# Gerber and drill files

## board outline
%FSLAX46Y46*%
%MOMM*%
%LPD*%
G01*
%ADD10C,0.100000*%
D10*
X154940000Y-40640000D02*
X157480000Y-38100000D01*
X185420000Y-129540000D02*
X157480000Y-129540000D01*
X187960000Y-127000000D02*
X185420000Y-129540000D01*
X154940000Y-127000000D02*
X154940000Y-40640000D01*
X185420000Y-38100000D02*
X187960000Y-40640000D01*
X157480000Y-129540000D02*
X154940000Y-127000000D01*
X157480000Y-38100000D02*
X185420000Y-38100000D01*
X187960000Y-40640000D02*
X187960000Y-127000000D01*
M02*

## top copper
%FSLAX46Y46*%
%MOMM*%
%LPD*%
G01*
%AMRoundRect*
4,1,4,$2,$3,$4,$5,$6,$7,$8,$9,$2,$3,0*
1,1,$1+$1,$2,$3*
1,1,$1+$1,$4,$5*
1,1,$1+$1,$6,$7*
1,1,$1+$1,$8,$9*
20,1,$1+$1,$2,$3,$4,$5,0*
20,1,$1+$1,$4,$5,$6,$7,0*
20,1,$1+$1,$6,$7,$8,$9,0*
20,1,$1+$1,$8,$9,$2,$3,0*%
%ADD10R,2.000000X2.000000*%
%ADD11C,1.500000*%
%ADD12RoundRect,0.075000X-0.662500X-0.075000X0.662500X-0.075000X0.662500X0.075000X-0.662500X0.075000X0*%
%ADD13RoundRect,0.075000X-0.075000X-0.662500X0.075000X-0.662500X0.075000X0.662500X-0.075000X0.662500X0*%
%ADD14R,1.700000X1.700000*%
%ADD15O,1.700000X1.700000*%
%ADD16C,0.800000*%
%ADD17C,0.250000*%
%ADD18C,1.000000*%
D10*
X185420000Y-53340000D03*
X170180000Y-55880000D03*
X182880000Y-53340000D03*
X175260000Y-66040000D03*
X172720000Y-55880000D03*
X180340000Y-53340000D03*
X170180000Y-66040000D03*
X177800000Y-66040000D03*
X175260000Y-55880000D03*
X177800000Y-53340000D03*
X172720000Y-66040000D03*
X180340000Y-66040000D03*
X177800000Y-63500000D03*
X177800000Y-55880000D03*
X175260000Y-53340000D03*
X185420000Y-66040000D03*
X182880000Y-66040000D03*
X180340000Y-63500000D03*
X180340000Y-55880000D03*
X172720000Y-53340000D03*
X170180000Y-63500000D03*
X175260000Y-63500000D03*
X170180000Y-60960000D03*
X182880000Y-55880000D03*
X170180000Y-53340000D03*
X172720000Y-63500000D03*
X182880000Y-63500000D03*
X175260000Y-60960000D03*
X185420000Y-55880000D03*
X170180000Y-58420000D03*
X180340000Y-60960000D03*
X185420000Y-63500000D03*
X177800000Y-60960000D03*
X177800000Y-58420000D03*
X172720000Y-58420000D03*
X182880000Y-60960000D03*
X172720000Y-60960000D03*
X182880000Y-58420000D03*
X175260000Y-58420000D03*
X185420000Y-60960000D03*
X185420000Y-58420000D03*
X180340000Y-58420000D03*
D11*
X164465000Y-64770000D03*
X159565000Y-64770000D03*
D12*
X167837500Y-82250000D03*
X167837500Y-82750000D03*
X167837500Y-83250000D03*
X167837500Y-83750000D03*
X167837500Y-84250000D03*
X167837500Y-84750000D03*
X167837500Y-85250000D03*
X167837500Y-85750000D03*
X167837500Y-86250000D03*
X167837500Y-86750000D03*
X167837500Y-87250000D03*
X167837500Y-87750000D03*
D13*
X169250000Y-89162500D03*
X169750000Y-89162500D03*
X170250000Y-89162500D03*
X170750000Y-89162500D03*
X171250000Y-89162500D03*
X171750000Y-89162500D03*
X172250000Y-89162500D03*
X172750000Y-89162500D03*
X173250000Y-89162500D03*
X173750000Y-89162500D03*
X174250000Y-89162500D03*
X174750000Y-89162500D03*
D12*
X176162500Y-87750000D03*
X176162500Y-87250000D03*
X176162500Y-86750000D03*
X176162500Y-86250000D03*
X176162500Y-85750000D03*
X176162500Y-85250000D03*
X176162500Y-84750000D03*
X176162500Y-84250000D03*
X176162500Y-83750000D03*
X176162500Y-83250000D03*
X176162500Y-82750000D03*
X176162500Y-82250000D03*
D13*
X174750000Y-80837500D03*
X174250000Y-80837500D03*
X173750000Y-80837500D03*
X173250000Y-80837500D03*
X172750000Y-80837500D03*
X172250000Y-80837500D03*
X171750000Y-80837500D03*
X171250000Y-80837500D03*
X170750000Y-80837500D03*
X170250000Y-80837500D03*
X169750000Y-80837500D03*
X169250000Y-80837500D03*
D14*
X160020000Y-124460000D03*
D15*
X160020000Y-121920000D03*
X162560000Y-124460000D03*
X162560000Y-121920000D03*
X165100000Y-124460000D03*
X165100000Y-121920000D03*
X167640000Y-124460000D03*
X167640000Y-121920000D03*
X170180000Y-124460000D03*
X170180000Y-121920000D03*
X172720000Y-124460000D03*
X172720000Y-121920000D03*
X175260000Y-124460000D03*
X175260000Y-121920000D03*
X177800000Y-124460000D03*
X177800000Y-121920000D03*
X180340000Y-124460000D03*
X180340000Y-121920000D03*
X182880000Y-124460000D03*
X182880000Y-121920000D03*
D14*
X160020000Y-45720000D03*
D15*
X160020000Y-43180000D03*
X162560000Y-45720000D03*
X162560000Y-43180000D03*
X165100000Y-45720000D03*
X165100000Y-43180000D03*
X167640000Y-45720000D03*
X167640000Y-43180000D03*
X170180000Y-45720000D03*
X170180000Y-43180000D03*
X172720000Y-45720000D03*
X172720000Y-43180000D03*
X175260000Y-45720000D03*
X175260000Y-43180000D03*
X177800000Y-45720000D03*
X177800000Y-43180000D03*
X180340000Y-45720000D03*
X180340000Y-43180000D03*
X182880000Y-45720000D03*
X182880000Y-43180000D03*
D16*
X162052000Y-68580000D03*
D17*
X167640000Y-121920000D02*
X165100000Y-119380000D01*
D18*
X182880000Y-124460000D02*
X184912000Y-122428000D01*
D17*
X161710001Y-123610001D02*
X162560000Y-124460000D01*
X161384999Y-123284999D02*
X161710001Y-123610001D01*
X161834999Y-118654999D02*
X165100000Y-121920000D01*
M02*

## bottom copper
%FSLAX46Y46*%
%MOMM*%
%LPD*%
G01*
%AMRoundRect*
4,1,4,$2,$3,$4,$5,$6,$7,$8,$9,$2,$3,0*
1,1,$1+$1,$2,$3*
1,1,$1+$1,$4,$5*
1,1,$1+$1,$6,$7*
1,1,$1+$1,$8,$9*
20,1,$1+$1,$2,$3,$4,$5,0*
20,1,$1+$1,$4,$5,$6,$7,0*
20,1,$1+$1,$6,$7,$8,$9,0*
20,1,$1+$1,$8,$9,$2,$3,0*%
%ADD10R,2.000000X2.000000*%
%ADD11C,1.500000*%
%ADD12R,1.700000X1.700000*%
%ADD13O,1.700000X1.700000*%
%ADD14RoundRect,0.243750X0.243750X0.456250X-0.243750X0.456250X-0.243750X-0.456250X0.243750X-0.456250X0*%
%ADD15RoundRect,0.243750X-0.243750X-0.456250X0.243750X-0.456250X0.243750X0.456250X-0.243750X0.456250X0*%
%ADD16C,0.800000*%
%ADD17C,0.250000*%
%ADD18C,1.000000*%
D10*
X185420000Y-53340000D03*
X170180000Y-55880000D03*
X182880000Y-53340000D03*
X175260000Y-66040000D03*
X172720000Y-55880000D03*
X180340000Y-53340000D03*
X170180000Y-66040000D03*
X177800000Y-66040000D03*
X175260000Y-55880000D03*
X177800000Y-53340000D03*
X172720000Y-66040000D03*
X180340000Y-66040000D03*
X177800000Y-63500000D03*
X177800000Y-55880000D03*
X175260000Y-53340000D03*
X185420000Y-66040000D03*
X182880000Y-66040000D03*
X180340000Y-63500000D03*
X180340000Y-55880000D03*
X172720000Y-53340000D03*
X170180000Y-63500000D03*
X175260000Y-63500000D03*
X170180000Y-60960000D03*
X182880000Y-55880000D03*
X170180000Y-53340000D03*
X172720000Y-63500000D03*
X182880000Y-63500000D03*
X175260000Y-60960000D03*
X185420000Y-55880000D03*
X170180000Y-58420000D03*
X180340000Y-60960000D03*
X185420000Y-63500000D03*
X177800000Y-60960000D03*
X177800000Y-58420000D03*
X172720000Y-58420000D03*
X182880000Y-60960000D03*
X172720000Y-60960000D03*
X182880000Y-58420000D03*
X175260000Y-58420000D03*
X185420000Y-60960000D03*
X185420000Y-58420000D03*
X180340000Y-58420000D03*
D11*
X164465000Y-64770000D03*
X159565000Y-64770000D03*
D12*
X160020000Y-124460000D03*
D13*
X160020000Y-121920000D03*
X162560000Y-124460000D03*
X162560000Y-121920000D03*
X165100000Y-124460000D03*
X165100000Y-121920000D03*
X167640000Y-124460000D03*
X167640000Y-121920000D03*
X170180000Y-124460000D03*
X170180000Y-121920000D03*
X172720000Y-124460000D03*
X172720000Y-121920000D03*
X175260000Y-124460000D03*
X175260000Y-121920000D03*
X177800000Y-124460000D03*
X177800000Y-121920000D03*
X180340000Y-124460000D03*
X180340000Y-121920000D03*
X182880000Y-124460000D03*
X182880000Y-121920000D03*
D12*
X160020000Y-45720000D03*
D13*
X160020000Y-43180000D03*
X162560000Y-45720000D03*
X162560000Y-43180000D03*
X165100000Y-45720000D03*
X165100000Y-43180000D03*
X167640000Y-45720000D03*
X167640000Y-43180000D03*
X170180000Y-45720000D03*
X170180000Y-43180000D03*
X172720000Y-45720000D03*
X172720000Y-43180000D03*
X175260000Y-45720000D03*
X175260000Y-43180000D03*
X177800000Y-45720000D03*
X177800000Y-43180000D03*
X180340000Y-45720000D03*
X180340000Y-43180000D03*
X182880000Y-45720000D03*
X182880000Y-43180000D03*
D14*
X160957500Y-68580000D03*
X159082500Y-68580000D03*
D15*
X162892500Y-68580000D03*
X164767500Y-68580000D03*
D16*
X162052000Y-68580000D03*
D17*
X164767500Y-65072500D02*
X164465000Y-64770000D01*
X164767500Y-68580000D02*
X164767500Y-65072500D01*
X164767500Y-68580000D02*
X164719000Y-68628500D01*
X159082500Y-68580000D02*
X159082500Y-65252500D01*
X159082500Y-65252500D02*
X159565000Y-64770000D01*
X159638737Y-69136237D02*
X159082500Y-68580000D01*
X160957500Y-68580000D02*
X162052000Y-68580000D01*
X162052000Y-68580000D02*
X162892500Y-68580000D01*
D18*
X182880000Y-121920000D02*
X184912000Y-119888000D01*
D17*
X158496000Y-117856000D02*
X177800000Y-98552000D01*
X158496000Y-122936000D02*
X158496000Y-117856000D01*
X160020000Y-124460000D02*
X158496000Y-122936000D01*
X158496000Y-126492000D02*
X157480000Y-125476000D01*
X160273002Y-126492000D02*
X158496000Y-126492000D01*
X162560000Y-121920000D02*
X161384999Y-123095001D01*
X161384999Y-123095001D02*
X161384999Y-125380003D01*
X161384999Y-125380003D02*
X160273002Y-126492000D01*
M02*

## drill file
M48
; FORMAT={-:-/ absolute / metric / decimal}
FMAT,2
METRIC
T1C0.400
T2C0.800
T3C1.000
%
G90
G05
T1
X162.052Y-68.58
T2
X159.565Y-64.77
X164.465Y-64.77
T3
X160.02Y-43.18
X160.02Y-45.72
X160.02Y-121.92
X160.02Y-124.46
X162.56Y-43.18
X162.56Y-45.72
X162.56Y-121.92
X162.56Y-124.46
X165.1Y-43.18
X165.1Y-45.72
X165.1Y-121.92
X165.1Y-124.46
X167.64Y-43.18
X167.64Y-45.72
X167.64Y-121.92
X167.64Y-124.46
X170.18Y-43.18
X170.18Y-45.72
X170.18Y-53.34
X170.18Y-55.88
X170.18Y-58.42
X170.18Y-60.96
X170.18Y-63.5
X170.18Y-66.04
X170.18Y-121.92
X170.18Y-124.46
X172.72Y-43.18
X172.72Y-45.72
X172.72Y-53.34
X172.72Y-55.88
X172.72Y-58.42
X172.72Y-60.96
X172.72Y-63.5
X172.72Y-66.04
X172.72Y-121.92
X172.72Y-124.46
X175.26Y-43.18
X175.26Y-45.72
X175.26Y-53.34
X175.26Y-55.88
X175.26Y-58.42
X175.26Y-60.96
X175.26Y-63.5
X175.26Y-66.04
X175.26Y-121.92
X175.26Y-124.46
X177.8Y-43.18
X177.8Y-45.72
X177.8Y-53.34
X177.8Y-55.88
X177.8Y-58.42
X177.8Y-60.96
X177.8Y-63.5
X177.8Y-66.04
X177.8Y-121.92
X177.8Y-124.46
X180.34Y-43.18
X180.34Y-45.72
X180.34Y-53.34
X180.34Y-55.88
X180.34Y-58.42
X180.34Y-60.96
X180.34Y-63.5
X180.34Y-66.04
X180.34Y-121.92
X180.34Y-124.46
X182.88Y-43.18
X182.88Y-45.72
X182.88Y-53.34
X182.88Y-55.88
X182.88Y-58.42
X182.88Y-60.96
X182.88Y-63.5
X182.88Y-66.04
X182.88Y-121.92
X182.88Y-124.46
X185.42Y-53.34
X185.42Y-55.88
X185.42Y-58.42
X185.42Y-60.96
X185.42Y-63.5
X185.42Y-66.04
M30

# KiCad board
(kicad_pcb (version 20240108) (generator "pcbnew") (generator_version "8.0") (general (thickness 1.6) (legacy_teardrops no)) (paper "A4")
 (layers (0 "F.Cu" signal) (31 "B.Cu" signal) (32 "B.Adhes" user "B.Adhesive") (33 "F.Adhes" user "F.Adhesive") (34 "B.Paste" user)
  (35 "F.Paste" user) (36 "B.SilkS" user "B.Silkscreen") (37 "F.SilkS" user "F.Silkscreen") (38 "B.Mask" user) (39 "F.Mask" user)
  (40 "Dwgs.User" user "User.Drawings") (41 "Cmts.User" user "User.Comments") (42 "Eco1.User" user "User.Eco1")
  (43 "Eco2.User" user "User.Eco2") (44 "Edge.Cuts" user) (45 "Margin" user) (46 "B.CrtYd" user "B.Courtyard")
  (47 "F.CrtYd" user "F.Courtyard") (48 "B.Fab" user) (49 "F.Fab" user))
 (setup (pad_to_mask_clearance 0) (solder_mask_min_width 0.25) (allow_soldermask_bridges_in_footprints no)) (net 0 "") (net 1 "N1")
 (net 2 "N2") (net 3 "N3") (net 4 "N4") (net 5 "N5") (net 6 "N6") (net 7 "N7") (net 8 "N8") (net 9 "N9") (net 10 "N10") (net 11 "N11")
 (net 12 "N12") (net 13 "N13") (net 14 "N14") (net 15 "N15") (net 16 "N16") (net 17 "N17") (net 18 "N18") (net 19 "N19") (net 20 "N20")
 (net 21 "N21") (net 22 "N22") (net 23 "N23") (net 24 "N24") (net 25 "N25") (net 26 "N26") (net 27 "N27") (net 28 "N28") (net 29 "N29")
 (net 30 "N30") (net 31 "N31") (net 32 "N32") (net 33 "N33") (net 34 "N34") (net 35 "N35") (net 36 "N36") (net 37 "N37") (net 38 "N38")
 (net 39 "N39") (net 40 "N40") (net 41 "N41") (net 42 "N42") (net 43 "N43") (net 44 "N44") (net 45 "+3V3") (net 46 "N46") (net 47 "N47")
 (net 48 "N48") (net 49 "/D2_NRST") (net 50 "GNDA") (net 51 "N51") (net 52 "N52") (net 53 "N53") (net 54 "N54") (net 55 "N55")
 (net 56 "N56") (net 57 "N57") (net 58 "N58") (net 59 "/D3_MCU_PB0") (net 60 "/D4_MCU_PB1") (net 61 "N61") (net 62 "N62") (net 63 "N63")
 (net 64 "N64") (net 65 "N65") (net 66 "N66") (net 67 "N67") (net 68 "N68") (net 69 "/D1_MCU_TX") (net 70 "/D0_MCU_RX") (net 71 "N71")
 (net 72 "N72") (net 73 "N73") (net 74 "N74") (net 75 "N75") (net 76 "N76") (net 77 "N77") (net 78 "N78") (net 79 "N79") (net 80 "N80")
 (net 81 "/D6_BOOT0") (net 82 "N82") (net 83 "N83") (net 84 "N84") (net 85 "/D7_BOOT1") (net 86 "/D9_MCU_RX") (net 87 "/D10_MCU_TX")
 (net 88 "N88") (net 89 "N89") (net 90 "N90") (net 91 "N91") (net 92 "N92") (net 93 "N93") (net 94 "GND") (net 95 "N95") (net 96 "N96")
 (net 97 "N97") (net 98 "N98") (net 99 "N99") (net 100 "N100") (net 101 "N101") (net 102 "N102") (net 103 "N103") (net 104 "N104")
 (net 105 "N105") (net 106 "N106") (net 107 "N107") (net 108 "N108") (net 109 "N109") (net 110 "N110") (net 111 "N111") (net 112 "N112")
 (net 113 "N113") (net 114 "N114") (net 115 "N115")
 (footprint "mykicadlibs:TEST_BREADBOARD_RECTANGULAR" (layer "F.Cu") (at 185.42 53.34)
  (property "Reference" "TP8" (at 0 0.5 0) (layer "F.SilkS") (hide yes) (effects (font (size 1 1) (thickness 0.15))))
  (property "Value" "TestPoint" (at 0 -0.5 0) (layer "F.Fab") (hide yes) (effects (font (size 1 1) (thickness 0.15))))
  (pad "1" thru_hole rect (at 0 0) (size 2 2) (drill 1) (layers "*.Cu" "*.Mask") (remove_unused_layers no) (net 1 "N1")))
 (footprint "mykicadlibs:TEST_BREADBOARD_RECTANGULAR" (layer "F.Cu") (at 170.18 55.88)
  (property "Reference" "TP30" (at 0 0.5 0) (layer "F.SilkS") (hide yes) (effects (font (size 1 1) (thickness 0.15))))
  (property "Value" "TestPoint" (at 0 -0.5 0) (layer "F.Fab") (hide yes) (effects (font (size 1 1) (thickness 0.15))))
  (pad "1" thru_hole rect (at 0 0) (size 2 2) (drill 1) (layers "*.Cu" "*.Mask") (remove_unused_layers no) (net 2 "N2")))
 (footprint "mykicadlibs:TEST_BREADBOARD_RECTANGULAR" (layer "F.Cu") (at 182.88 53.34)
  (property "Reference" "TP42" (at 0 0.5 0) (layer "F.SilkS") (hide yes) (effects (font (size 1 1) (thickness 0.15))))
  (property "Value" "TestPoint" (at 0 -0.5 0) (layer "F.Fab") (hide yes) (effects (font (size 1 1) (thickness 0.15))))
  (pad "1" thru_hole rect (at 0 0) (size 2 2) (drill 1) (layers "*.Cu" "*.Mask") (remove_unused_layers no) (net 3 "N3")))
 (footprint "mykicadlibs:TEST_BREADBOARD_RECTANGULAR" (layer "F.Cu") (at 175.26 66.04)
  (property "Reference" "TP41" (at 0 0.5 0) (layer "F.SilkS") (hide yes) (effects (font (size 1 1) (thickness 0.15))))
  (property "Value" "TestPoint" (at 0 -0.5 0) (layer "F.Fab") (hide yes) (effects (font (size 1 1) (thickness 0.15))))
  (pad "1" thru_hole rect (at 0 0) (size 2 2) (drill 1) (layers "*.Cu" "*.Mask") (remove_unused_layers no) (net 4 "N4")))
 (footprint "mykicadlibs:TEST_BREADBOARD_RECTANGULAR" (layer "F.Cu") (at 172.72 55.88)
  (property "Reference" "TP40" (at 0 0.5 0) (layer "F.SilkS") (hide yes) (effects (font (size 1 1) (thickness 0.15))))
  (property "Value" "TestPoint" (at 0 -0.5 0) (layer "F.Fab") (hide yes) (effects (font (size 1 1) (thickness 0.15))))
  (pad "1" thru_hole rect (at 0 0) (size 2 2) (drill 1) (layers "*.Cu" "*.Mask") (remove_unused_layers no) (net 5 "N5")))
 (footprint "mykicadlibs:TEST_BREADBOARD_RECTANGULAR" (layer "F.Cu") (at 180.34 53.34)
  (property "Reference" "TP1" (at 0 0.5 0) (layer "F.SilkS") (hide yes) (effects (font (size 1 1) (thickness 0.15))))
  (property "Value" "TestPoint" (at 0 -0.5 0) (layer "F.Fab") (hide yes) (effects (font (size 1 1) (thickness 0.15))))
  (pad "1" thru_hole rect (at 0 0) (size 2 2) (drill 1) (layers "*.Cu" "*.Mask") (remove_unused_layers no) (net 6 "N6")))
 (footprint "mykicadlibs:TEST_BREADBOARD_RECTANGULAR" (layer "F.Cu") (at 170.18 66.04)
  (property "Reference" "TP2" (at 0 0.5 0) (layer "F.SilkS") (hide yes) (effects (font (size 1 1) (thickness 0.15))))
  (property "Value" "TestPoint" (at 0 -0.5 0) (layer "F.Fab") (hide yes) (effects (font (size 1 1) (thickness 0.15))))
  (pad "1" thru_hole rect (at 0 0) (size 2 2) (drill 1) (layers "*.Cu" "*.Mask") (remove_unused_layers no) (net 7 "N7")))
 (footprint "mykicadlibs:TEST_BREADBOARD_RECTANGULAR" (layer "F.Cu") (at 177.8 66.04)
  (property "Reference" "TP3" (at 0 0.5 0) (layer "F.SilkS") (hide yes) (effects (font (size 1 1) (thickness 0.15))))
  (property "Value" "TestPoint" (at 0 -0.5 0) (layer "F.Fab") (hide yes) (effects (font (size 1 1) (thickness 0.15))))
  (pad "1" thru_hole rect (at 0 0) (size 2 2) (drill 1) (layers "*.Cu" "*.Mask") (remove_unused_layers no) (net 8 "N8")))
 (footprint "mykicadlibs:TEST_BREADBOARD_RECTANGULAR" (layer "F.Cu") (at 175.26 55.88)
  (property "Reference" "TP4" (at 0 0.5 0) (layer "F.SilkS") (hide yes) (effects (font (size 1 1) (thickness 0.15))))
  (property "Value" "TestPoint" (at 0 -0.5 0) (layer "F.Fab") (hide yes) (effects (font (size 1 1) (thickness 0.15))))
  (pad "1" thru_hole rect (at 0 0) (size 2 2) (drill 1) (layers "*.Cu" "*.Mask") (remove_unused_layers no) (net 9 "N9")))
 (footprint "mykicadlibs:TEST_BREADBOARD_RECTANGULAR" (layer "F.Cu") (at 177.8 53.34)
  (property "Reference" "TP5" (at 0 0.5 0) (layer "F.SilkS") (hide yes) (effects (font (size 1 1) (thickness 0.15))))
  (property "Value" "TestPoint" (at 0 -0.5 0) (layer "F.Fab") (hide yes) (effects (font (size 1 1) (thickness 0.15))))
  (pad "1" thru_hole rect (at 0 0) (size 2 2) (drill 1) (layers "*.Cu" "*.Mask") (remove_unused_layers no) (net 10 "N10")))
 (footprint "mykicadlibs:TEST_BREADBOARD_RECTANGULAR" (layer "F.Cu") (at 172.72 66.04)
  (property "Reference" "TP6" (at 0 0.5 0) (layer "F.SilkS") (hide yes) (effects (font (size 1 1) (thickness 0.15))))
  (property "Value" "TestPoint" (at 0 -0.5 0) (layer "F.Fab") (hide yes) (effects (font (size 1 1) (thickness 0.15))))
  (pad "1" thru_hole rect (at 0 0) (size 2 2) (drill 1) (layers "*.Cu" "*.Mask") (remove_unused_layers no) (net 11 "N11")))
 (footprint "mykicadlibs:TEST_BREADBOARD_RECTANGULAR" (layer "F.Cu") (at 180.34 66.04)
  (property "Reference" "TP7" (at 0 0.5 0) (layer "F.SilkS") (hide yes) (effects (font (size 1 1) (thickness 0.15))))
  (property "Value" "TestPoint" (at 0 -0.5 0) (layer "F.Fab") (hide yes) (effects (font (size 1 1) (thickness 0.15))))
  (pad "1" thru_hole rect (at 0 0) (size 2 2) (drill 1) (layers "*.Cu" "*.Mask") (remove_unused_layers no) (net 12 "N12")))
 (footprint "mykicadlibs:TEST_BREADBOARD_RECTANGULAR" (layer "F.Cu") (at 177.8 63.5)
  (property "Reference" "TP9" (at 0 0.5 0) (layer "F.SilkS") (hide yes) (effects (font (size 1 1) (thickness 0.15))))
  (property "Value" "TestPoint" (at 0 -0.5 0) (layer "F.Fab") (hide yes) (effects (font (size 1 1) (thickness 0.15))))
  (pad "1" thru_hole rect (at 0 0) (size 2 2) (drill 1) (layers "*.Cu" "*.Mask") (remove_unused_layers no) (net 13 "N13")))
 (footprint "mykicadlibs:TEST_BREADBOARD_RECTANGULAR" (layer "F.Cu") (at 177.8 55.88)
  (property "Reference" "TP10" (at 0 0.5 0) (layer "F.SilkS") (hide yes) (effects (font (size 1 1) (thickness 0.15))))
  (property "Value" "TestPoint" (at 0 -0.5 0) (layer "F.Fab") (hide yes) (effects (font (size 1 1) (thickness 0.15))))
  (pad "1" thru_hole rect (at 0 0) (size 2 2) (drill 1) (layers "*.Cu" "*.Mask") (remove_unused_layers no) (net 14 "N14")))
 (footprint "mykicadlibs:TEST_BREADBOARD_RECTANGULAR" (layer "F.Cu") (at 175.26 53.34)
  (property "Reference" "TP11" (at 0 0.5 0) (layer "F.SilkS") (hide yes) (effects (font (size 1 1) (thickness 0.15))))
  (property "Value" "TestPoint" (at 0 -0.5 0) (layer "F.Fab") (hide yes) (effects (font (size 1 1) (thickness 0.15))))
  (pad "1" thru_hole rect (at 0 0) (size 2 2) (drill 1) (layers "*.Cu" "*.Mask") (remove_unused_layers no) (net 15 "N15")))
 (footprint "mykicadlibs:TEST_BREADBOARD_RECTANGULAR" (layer "F.Cu") (at 185.42 66.04)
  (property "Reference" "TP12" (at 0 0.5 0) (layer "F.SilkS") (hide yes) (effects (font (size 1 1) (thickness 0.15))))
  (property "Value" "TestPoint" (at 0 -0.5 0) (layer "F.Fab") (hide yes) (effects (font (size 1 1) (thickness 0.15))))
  (pad "1" thru_hole rect (at 0 0) (size 2 2) (drill 1) (layers "*.Cu" "*.Mask") (remove_unused_layers no) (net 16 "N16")))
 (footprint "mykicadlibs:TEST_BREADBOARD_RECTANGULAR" (layer "F.Cu") (at 182.88 66.04)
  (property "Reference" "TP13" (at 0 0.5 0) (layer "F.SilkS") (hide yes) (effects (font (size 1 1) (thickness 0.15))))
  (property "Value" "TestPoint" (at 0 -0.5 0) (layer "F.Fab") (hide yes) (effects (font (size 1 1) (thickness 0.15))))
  (pad "1" thru_hole rect (at 0 0) (size 2 2) (drill 1) (layers "*.Cu" "*.Mask") (remove_unused_layers no) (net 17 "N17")))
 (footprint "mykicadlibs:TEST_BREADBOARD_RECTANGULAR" (layer "F.Cu") (at 180.34 63.5)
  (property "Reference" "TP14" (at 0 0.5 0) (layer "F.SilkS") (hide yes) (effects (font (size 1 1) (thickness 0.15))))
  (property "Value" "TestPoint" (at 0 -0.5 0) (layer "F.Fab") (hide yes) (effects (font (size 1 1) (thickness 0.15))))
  (pad "1" thru_hole rect (at 0 0) (size 2 2) (drill 1) (layers "*.Cu" "*.Mask") (remove_unused_layers no) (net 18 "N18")))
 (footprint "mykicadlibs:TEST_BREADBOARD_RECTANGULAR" (layer "F.Cu") (at 180.34 55.88)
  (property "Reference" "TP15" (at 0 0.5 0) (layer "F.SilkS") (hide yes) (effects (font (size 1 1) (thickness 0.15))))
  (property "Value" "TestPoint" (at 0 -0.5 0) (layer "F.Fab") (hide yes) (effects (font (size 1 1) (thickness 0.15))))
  (pad "1" thru_hole rect (at 0 0) (size 2 2) (drill 1) (layers "*.Cu" "*.Mask") (remove_unused_layers no) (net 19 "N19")))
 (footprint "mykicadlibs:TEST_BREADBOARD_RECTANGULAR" (layer "F.Cu") (at 172.72 53.34)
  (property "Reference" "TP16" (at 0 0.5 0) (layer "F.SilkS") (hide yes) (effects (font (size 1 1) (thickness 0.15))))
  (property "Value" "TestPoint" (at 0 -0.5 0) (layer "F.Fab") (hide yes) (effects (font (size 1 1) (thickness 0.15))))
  (pad "1" thru_hole rect (at 0 0) (size 2 2) (drill 1) (layers "*.Cu" "*.Mask") (remove_unused_layers no) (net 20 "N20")))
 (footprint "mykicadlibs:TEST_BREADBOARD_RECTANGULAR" (layer "F.Cu") (at 170.18 63.5)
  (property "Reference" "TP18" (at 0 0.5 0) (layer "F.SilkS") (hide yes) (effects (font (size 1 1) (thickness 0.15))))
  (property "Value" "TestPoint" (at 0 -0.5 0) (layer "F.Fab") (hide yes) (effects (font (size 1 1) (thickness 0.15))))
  (pad "1" thru_hole rect (at 0 0) (size 2 2) (drill 1) (layers "*.Cu" "*.Mask") (remove_unused_layers no) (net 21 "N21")))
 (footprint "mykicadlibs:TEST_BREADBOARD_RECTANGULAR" (layer "F.Cu") (at 175.26 63.5)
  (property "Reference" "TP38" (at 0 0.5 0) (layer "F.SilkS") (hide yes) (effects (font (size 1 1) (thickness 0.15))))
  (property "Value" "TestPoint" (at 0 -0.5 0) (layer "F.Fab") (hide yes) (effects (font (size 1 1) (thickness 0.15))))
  (pad "1" thru_hole rect (at 0 0) (size 2 2) (drill 1) (layers "*.Cu" "*.Mask") (remove_unused_layers no) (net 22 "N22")))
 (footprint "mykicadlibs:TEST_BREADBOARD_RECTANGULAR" (layer "F.Cu") (at 170.18 60.96)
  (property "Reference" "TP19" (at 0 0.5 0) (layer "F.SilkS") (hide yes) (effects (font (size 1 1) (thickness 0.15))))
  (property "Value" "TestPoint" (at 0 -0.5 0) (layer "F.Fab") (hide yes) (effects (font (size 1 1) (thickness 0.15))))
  (pad "1" thru_hole rect (at 0 0) (size 2 2) (drill 1) (layers "*.Cu" "*.Mask") (remove_unused_layers no) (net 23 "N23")))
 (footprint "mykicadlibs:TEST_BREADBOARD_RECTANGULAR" (layer "F.Cu") (at 182.88 55.88)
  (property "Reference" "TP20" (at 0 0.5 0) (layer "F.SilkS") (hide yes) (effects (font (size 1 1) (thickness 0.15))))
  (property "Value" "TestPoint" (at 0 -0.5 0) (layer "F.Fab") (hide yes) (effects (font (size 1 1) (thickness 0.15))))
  (pad "1" thru_hole rect (at 0 0) (size 2 2) (drill 1) (layers "*.Cu" "*.Mask") (remove_unused_layers no) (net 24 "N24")))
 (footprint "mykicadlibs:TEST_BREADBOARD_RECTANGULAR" (layer "F.Cu") (at 170.18 53.34)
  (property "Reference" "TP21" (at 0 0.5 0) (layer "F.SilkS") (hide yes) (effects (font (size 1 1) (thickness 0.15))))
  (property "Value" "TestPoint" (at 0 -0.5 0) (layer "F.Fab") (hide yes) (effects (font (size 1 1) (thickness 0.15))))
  (pad "1" thru_hole rect (at 0 0) (size 2 2) (drill 1) (layers "*.Cu" "*.Mask") (remove_unused_layers no) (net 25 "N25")))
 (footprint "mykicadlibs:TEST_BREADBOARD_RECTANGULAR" (layer "F.Cu") (at 172.72 63.5)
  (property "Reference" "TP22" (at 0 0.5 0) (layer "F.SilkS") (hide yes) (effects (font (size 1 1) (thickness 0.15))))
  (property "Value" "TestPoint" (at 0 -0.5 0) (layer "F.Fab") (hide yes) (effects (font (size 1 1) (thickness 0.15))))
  (pad "1" thru_hole rect (at 0 0) (size 2 2) (drill 1) (layers "*.Cu" "*.Mask") (remove_unused_layers no) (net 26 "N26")))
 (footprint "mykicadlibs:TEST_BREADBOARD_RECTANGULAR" (layer "F.Cu") (at 182.88 63.5)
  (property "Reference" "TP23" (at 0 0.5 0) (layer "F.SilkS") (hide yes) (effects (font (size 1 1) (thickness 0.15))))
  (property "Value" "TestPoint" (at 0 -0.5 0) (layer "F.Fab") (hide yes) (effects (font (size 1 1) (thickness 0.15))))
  (pad "1" thru_hole rect (at 0 0) (size 2 2) (drill 1) (layers "*.Cu" "*.Mask") (remove_unused_layers no) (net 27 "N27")))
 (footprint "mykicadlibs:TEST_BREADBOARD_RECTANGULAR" (layer "F.Cu") (at 175.26 60.96)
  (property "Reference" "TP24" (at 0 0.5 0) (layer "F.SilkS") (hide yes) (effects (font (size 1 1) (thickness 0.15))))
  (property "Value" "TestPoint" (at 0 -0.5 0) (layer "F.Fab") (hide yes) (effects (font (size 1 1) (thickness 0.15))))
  (pad "1" thru_hole rect (at 0 0) (size 2 2) (drill 1) (layers "*.Cu" "*.Mask") (remove_unused_layers no) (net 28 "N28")))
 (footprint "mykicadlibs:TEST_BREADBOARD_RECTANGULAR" (layer "F.Cu") (at 185.42 55.88)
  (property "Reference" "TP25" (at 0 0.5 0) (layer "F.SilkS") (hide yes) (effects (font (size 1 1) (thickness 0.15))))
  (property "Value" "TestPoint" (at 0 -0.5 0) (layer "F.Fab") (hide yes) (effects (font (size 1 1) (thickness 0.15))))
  (pad "1" thru_hole rect (at 0 0) (size 2 2) (drill 1) (layers "*.Cu" "*.Mask") (remove_unused_layers no) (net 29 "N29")))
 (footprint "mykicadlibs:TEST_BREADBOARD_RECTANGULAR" (layer "F.Cu") (at 170.18 58.42)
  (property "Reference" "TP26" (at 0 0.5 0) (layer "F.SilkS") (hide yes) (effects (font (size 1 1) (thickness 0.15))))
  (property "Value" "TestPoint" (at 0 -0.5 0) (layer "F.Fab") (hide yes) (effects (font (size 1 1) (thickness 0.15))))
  (pad "1" thru_hole rect (at 0 0) (size 2 2) (drill 1) (layers "*.Cu" "*.Mask") (remove_unused_layers no) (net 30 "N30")))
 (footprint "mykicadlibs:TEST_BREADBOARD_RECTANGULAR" (layer "F.Cu") (at 180.34 60.96)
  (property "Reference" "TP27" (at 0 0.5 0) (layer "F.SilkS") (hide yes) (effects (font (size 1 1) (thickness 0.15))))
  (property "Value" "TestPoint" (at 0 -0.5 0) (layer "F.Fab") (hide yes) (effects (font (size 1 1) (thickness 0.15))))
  (pad "1" thru_hole rect (at 0 0) (size 2 2) (drill 1) (layers "*.Cu" "*.Mask") (remove_unused_layers no) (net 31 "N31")))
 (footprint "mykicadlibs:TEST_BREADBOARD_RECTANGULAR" (layer "F.Cu") (at 185.42 63.5)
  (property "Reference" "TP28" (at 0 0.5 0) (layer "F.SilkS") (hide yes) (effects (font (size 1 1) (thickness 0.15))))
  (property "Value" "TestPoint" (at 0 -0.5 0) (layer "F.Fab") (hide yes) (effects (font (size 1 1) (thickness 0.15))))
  (pad "1" thru_hole rect (at 0 0) (size 2 2) (drill 1) (layers "*.Cu" "*.Mask") (remove_unused_layers no) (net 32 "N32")))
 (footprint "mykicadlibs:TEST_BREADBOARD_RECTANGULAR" (layer "F.Cu") (at 177.8 60.96)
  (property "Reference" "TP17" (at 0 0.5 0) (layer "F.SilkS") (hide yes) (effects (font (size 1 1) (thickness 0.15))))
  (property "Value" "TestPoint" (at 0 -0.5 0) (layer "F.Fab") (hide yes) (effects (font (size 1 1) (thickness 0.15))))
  (pad "1" thru_hole rect (at 0 0) (size 2 2) (drill 1) (layers "*.Cu" "*.Mask") (remove_unused_layers no) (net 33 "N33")))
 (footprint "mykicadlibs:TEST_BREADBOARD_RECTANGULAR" (layer "F.Cu") (at 177.8 58.42)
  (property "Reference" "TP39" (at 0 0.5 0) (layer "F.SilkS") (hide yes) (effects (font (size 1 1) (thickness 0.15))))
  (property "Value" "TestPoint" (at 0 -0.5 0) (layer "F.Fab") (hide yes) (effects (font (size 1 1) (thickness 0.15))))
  (pad "1" thru_hole rect (at 0 0) (size 2 2) (drill 1) (layers "*.Cu" "*.Mask") (remove_unused_layers no) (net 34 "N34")))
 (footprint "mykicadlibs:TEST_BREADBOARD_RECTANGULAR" (layer "F.Cu") (at 172.72 58.42)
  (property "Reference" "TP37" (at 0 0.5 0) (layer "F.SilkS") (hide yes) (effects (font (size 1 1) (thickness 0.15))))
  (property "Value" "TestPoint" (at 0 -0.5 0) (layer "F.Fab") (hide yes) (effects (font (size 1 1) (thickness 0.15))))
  (pad "1" thru_hole rect (at 0 0) (size 2 2) (drill 1) (layers "*.Cu" "*.Mask") (remove_unused_layers no) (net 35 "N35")))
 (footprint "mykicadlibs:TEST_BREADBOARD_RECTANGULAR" (layer "F.Cu") (at 182.88 60.96)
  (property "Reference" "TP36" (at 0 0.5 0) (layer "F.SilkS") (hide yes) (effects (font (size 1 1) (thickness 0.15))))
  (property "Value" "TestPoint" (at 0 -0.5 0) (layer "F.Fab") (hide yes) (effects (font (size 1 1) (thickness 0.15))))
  (pad "1" thru_hole rect (at 0 0) (size 2 2) (drill 1) (layers "*.Cu" "*.Mask") (remove_unused_layers no) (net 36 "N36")))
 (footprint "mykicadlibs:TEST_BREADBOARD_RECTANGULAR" (layer "F.Cu") (at 172.72 60.96)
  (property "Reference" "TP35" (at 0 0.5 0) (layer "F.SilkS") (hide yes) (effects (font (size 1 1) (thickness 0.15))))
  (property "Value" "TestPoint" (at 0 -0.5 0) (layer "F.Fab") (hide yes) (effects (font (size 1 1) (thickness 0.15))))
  (pad "1" thru_hole rect (at 0 0) (size 2 2) (drill 1) (layers "*.Cu" "*.Mask") (remove_unused_layers no) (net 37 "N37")))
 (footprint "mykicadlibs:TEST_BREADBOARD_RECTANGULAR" (layer "F.Cu") (at 182.88 58.42)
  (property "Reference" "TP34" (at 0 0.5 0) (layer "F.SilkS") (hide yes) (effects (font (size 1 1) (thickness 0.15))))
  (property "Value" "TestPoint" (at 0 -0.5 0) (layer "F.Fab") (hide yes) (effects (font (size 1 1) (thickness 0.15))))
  (pad "1" thru_hole rect (at 0 0) (size 2 2) (drill 1) (layers "*.Cu" "*.Mask") (remove_unused_layers no) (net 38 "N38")))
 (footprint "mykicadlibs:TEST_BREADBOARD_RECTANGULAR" (layer "F.Cu") (at 175.26 58.42)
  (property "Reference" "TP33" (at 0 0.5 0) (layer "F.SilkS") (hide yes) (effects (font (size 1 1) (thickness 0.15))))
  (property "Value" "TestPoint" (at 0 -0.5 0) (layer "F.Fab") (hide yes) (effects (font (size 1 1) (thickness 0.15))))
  (pad "1" thru_hole rect (at 0 0) (size 2 2) (drill 1) (layers "*.Cu" "*.Mask") (remove_unused_layers no) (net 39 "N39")))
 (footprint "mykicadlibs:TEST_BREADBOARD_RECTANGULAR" (layer "F.Cu") (at 185.42 60.96)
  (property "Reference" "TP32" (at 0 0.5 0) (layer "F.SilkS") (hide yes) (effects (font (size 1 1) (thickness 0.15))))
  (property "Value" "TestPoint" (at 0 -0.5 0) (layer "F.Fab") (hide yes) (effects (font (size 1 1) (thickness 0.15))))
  (pad "1" thru_hole rect (at 0 0) (size 2 2) (drill 1) (layers "*.Cu" "*.Mask") (remove_unused_layers no) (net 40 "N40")))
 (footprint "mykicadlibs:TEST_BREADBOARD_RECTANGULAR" (layer "F.Cu") (at 185.42 58.42)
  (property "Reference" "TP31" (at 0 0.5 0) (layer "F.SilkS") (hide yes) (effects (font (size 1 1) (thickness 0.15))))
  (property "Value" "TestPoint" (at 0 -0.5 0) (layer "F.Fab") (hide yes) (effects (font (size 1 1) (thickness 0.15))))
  (pad "1" thru_hole rect (at 0 0) (size 2 2) (drill 1) (layers "*.Cu" "*.Mask") (remove_unused_layers no) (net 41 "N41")))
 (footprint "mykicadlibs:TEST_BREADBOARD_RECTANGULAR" (layer "F.Cu") (at 180.34 58.42)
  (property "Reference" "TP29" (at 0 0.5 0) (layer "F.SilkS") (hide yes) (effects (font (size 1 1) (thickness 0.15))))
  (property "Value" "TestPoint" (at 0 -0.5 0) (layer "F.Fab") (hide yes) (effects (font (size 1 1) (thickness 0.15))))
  (pad "1" thru_hole rect (at 0 0) (size 2 2) (drill 1) (layers "*.Cu" "*.Mask") (remove_unused_layers no) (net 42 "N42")))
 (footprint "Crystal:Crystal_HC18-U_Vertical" (layer "F.Cu") (at 164.465 64.77 180)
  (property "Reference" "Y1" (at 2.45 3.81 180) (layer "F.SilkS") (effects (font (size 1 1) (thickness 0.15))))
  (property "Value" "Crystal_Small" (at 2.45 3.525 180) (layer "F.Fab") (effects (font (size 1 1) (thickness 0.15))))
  (pad "1" thru_hole circle (at 0 0 180) (size 1.5 1.5) (drill 0.8) (layers "*.Cu" "*.Mask") (remove_unused_layers no) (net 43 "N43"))
  (pad "2" thru_hole circle (at 4.9 0 180) (size 1.5 1.5) (drill 0.8) (layers "*.Cu" "*.Mask") (remove_unused_layers no) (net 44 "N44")))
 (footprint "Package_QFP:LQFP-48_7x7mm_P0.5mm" (layer "F.Cu") (at 172 85)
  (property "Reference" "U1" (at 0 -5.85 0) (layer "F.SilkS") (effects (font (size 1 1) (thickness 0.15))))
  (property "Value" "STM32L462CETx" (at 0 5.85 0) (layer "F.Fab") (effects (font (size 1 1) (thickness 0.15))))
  (pad "1" smd roundrect (at -4.1625 -2.75) (size 1.475 0.3) (layers "F.Cu" "F.Paste" "F.Mask") (roundrect_rratio 0.25) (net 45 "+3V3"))
  (pad "2" smd roundrect (at -4.1625 -2.25) (size 1.475 0.3) (layers "F.Cu" "F.Paste" "F.Mask") (roundrect_rratio 0.25) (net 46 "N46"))
  (pad "3" smd roundrect (at -4.1625 -1.75) (size 1.475 0.3) (layers "F.Cu" "F.Paste" "F.Mask") (roundrect_rratio 0.25) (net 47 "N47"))
  (pad "4" smd roundrect (at -4.1625 -1.25) (size 1.475 0.3) (layers "F.Cu" "F.Paste" "F.Mask") (roundrect_rratio 0.25) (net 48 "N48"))
  (pad "5" smd roundrect (at -4.1625 -0.75) (size 1.475 0.3) (layers "F.Cu" "F.Paste" "F.Mask") (roundrect_rratio 0.25) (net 43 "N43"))
  (pad "6" smd roundrect (at -4.1625 -0.25) (size 1.475 0.3) (layers "F.Cu" "F.Paste" "F.Mask") (roundrect_rratio 0.25) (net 44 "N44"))
  (pad "7" smd roundrect (at -4.1625 0.25) (size 1.475 0.3) (layers "F.Cu" "F.Paste" "F.Mask") (roundrect_rratio 0.25) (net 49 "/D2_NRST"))
  (pad "8" smd roundrect (at -4.1625 0.75) (size 1.475 0.3) (layers "F.Cu" "F.Paste" "F.Mask") (roundrect_rratio 0.25) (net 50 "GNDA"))
  (pad "9" smd roundrect (at -4.1625 1.25) (size 1.475 0.3) (layers "F.Cu" "F.Paste" "F.Mask") (roundrect_rratio 0.25) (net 45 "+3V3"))
  (pad "10" smd roundrect (at -4.1625 1.75) (size 1.475 0.3) (layers "F.Cu" "F.Paste" "F.Mask") (roundrect_rratio 0.25) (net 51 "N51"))
  (pad "11" smd roundrect (at -4.1625 2.25) (size 1.475 0.3) (layers "F.Cu" "F.Paste" "F.Mask") (roundrect_rratio 0.25) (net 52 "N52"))
  (pad "12" smd roundrect (at -4.1625 2.75) (size 1.475 0.3) (layers "F.Cu" "F.Paste" "F.Mask") (roundrect_rratio 0.25) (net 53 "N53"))
  (pad "13" smd roundrect (at -2.75 4.1625) (size 0.3 1.475) (layers "F.Cu" "F.Paste" "F.Mask") (roundrect_rratio 0.25) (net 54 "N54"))
  (pad "14" smd roundrect (at -2.25 4.1625) (size 0.3 1.475) (layers "F.Cu" "F.Paste" "F.Mask") (roundrect_rratio 0.25) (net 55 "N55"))
  (pad "15" smd roundrect (at -1.75 4.1625) (size 0.3 1.475) (layers "F.Cu" "F.Paste" "F.Mask") (roundrect_rratio 0.25) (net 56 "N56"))
  (pad "16" smd roundrect (at -1.25 4.1625) (size 0.3 1.475) (layers "F.Cu" "F.Paste" "F.Mask") (roundrect_rratio 0.25) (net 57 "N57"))
  (pad "17" smd roundrect (at -0.75 4.1625) (size 0.3 1.475) (layers "F.Cu" "F.Paste" "F.Mask") (roundrect_rratio 0.25) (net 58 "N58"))
  (pad "18" smd roundrect (at -0.25 4.1625) (size 0.3 1.475) (layers "F.Cu" "F.Paste" "F.Mask") (roundrect_rratio 0.25)
   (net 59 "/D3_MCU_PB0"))
  (pad "19" smd roundrect (at 0.25 4.1625) (size 0.3 1.475) (layers "F.Cu" "F.Paste" "F.Mask") (roundrect_rratio 0.25)
   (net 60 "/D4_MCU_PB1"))
  (pad "20" smd roundrect (at 0.75 4.1625) (size 0.3 1.475) (layers "F.Cu" "F.Paste" "F.Mask") (roundrect_rratio 0.25) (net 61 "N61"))
  (pad "21" smd roundrect (at 1.25 4.1625) (size 0.3 1.475) (layers "F.Cu" "F.Paste" "F.Mask") (roundrect_rratio 0.25) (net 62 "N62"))
  (pad "22" smd roundrect (at 1.75 4.1625) (size 0.3 1.475) (layers "F.Cu" "F.Paste" "F.Mask") (roundrect_rratio 0.25) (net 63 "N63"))
  (pad "23" smd roundrect (at 2.25 4.1625) (size 0.3 1.475) (layers "F.Cu" "F.Paste" "F.Mask") (roundrect_rratio 0.25) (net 50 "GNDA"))
  (pad "24" smd roundrect (at 2.75 4.1625) (size 0.3 1.475) (layers "F.Cu" "F.Paste" "F.Mask") (roundrect_rratio 0.25) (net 45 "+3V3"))
  (pad "25" smd roundrect (at 4.1625 2.75) (size 1.475 0.3) (layers "F.Cu" "F.Paste" "F.Mask") (roundrect_rratio 0.25) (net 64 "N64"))
  (pad "26" smd roundrect (at 4.1625 2.25) (size 1.475 0.3) (layers "F.Cu" "F.Paste" "F.Mask") (roundrect_rratio 0.25) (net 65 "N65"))
  (pad "27" smd roundrect (at 4.1625 1.75) (size 1.475 0.3) (layers "F.Cu" "F.Paste" "F.Mask") (roundrect_rratio 0.25) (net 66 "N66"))
  (pad "28" smd roundrect (at 4.1625 1.25) (size 1.475 0.3) (layers "F.Cu" "F.Paste" "F.Mask") (roundrect_rratio 0.25) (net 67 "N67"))
  (pad "29" smd roundrect (at 4.1625 0.75) (size 1.475 0.3) (layers "F.Cu" "F.Paste" "F.Mask") (roundrect_rratio 0.25) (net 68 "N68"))
  (pad "30" smd roundrect (at 4.1625 0.25) (size 1.475 0.3) (layers "F.Cu" "F.Paste" "F.Mask") (roundrect_rratio 0.25) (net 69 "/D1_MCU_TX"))
  (pad "31" smd roundrect (at 4.1625 -0.25) (size 1.475 0.3) (layers "F.Cu" "F.Paste" "F.Mask") (roundrect_rratio 0.25)
   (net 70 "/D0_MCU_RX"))
  (pad "32" smd roundrect (at 4.1625 -0.75) (size 1.475 0.3) (layers "F.Cu" "F.Paste" "F.Mask") (roundrect_rratio 0.25) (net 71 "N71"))
  (pad "33" smd roundrect (at 4.1625 -1.25) (size 1.475 0.3) (layers "F.Cu" "F.Paste" "F.Mask") (roundrect_rratio 0.25) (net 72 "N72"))
  (pad "34" smd roundrect (at 4.1625 -1.75) (size 1.475 0.3) (layers "F.Cu" "F.Paste" "F.Mask") (roundrect_rratio 0.25) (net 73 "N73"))
  (pad "35" smd roundrect (at 4.1625 -2.25) (size 1.475 0.3) (layers "F.Cu" "F.Paste" "F.Mask") (roundrect_rratio 0.25) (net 50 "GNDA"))
  (pad "36" smd roundrect (at 4.1625 -2.75) (size 1.475 0.3) (layers "F.Cu" "F.Paste" "F.Mask") (roundrect_rratio 0.25) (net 45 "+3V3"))
  (pad "37" smd roundrect (at 2.75 -4.1625) (size 0.3 1.475) (layers "F.Cu" "F.Paste" "F.Mask") (roundrect_rratio 0.25) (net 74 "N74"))
  (pad "38" smd roundrect (at 2.25 -4.1625) (size 0.3 1.475) (layers "F.Cu" "F.Paste" "F.Mask") (roundrect_rratio 0.25) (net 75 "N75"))
  (pad "39" smd roundrect (at 1.75 -4.1625) (size 0.3 1.475) (layers "F.Cu" "F.Paste" "F.Mask") (roundrect_rratio 0.25) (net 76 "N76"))
  (pad "40" smd roundrect (at 1.25 -4.1625) (size 0.3 1.475) (layers "F.Cu" "F.Paste" "F.Mask") (roundrect_rratio 0.25) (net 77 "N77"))
  (pad "41" smd roundrect (at 0.75 -4.1625) (size 0.3 1.475) (layers "F.Cu" "F.Paste" "F.Mask") (roundrect_rratio 0.25) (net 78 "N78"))
  (pad "42" smd roundrect (at 0.25 -4.1625) (size 0.3 1.475) (layers "F.Cu" "F.Paste" "F.Mask") (roundrect_rratio 0.25) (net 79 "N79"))
  (pad "43" smd roundrect (at -0.25 -4.1625) (size 0.3 1.475) (layers "F.Cu" "F.Paste" "F.Mask") (roundrect_rratio 0.25) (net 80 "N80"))
  (pad "44" smd roundrect (at -0.75 -4.1625) (size 0.3 1.475) (layers "F.Cu" "F.Paste" "F.Mask") (roundrect_rratio 0.25)
   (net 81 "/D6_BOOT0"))
  (pad "45" smd roundrect (at -1.25 -4.1625) (size 0.3 1.475) (layers "F.Cu" "F.Paste" "F.Mask") (roundrect_rratio 0.25) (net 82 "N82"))
  (pad "46" smd roundrect (at -1.75 -4.1625) (size 0.3 1.475) (layers "F.Cu" "F.Paste" "F.Mask") (roundrect_rratio 0.25) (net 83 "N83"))
  (pad "47" smd roundrect (at -2.25 -4.1625) (size 0.3 1.475) (layers "F.Cu" "F.Paste" "F.Mask") (roundrect_rratio 0.25) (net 50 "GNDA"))
  (pad "48" smd roundrect (at -2.75 -4.1625) (size 0.3 1.475) (layers "F.Cu" "F.Paste" "F.Mask") (roundrect_rratio 0.25) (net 45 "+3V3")))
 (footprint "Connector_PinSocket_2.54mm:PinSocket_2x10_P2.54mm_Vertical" (layer "B.Cu") (at 160.02 124.46 -90)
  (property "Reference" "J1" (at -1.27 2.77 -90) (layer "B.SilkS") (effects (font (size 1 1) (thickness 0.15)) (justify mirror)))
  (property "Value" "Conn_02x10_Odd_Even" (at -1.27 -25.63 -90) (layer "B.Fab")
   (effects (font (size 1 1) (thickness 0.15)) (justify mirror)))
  (pad "1" thru_hole rect (at 0 0 270) (size 1.7 1.7) (drill 1) (layers "*.Cu" "*.Mask") (remove_unused_layers no) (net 69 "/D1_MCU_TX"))
  (pad "2" thru_hole oval (at -2.54 0 270) (size 1.7 1.7) (drill 1) (layers "*.Cu" "*.Mask") (remove_unused_layers no) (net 70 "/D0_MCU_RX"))
  (pad "3" thru_hole oval (at 0 -2.54 270) (size 1.7 1.7) (drill 1) (layers "*.Cu" "*.Mask") (remove_unused_layers no)
   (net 59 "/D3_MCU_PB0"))
  (pad "4" thru_hole oval (at -2.54 -2.54 270) (size 1.7 1.7) (drill 1) (layers "*.Cu" "*.Mask") (remove_unused_layers no)
   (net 49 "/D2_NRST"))
  (pad "5" thru_hole oval (at 0 -5.08 270) (size 1.7 1.7) (drill 1) (layers "*.Cu" "*.Mask") (remove_unused_layers no) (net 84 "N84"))
  (pad "6" thru_hole oval (at -2.54 -5.08 270) (size 1.7 1.7) (drill 1) (layers "*.Cu" "*.Mask") (remove_unused_layers no)
   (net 60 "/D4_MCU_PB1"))
  (pad "7" thru_hole oval (at 0 -7.62 270) (size 1.7 1.7) (drill 1) (layers "*.Cu" "*.Mask") (remove_unused_layers no) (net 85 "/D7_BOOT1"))
  (pad "8" thru_hole oval (at -2.54 -7.62 270) (size 1.7 1.7) (drill 1) (layers "*.Cu" "*.Mask") (remove_unused_layers no)
   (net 81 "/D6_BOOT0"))
  (pad "9" thru_hole oval (at 0 -10.16 270) (size 1.7 1.7) (drill 1) (layers "*.Cu" "*.Mask") (remove_unused_layers no)
   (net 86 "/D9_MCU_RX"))
  (pad "10" thru_hole oval (at -2.54 -10.16 270) (size 1.7 1.7) (drill 1) (layers "*.Cu" "*.Mask") (remove_unused_layers no)
   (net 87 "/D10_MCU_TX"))
  (pad "11" thru_hole oval (at 0 -12.7 270) (size 1.7 1.7) (drill 1) (layers "*.Cu" "*.Mask") (remove_unused_layers no) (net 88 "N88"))
  (pad "12" thru_hole oval (at -2.54 -12.7 270) (size 1.7 1.7) (drill 1) (layers "*.Cu" "*.Mask") (remove_unused_layers no) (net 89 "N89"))
  (pad "13" thru_hole oval (at 0 -15.24 270) (size 1.7 1.7) (drill 1) (layers "*.Cu" "*.Mask") (remove_unused_layers no) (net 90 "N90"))
  (pad "14" thru_hole oval (at -2.54 -15.24 270) (size 1.7 1.7) (drill 1) (layers "*.Cu" "*.Mask") (remove_unused_layers no) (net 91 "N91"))
  (pad "15" thru_hole oval (at 0 -17.78 270) (size 1.7 1.7) (drill 1) (layers "*.Cu" "*.Mask") (remove_unused_layers no) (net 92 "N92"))
  (pad "16" thru_hole oval (at -2.54 -17.78 270) (size 1.7 1.7) (drill 1) (layers "*.Cu" "*.Mask") (remove_unused_layers no) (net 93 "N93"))
  (pad "17" thru_hole oval (at 0 -20.32 270) (size 1.7 1.7) (drill 1) (layers "*.Cu" "*.Mask") (remove_unused_layers no) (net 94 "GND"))
  (pad "18" thru_hole oval (at -2.54 -20.32 270) (size 1.7 1.7) (drill 1) (layers "*.Cu" "*.Mask") (remove_unused_layers no) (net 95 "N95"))
  (pad "19" thru_hole oval (at 0 -22.86 270) (size 1.7 1.7) (drill 1) (layers "*.Cu" "*.Mask") (remove_unused_layers no) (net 50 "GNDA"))
  (pad "20" thru_hole oval (at -2.54 -22.86 270) (size 1.7 1.7) (drill 1) (layers "*.Cu" "*.Mask") (remove_unused_layers no) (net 45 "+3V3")))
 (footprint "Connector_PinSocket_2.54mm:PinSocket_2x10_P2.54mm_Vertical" (layer "B.Cu") (at 160.02 45.72 -90)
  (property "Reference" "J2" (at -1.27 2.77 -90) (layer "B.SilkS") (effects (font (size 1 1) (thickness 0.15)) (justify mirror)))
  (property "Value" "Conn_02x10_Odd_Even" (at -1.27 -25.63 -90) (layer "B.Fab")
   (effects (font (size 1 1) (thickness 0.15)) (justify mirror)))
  (pad "1" thru_hole rect (at 0 0 270) (size 1.7 1.7) (drill 1) (layers "*.Cu" "*.Mask") (remove_unused_layers no) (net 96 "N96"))
  (pad "2" thru_hole oval (at -2.54 0 270) (size 1.7 1.7) (drill 1) (layers "*.Cu" "*.Mask") (remove_unused_layers no) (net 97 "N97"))
  (pad "3" thru_hole oval (at 0 -2.54 270) (size 1.7 1.7) (drill 1) (layers "*.Cu" "*.Mask") (remove_unused_layers no) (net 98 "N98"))
  (pad "4" thru_hole oval (at -2.54 -2.54 270) (size 1.7 1.7) (drill 1) (layers "*.Cu" "*.Mask") (remove_unused_layers no) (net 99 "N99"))
  (pad "5" thru_hole oval (at 0 -5.08 270) (size 1.7 1.7) (drill 1) (layers "*.Cu" "*.Mask") (remove_unused_layers no) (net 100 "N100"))
  (pad "6" thru_hole oval (at -2.54 -5.08 270) (size 1.7 1.7) (drill 1) (layers "*.Cu" "*.Mask") (remove_unused_layers no) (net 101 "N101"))
  (pad "7" thru_hole oval (at 0 -7.62 270) (size 1.7 1.7) (drill 1) (layers "*.Cu" "*.Mask") (remove_unused_layers no) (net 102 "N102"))
  (pad "8" thru_hole oval (at -2.54 -7.62 270) (size 1.7 1.7) (drill 1) (layers "*.Cu" "*.Mask") (remove_unused_layers no) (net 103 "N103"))
  (pad "9" thru_hole oval (at 0 -10.16 270) (size 1.7 1.7) (drill 1) (layers "*.Cu" "*.Mask") (remove_unused_layers no) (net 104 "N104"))
  (pad "10" thru_hole oval (at -2.54 -10.16 270) (size 1.7 1.7) (drill 1) (layers "*.Cu" "*.Mask") (remove_unused_layers no)
   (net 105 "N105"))
  (pad "11" thru_hole oval (at 0 -12.7 270) (size 1.7 1.7) (drill 1) (layers "*.Cu" "*.Mask") (remove_unused_layers no) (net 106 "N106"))
  (pad "12" thru_hole oval (at -2.54 -12.7 270) (size 1.7 1.7) (drill 1) (layers "*.Cu" "*.Mask") (remove_unused_layers no) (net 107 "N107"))
  (pad "13" thru_hole oval (at 0 -15.24 270) (size 1.7 1.7) (drill 1) (layers "*.Cu" "*.Mask") (remove_unused_layers no) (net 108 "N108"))
  (pad "14" thru_hole oval (at -2.54 -15.24 270) (size 1.7 1.7) (drill 1) (layers "*.Cu" "*.Mask") (remove_unused_layers no)
   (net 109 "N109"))
  (pad "15" thru_hole oval (at 0 -17.78 270) (size 1.7 1.7) (drill 1) (layers "*.Cu" "*.Mask") (remove_unused_layers no) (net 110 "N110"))
  (pad "16" thru_hole oval (at -2.54 -17.78 270) (size 1.7 1.7) (drill 1) (layers "*.Cu" "*.Mask") (remove_unused_layers no)
   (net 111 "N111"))
  (pad "17" thru_hole oval (at 0 -20.32 270) (size 1.7 1.7) (drill 1) (layers "*.Cu" "*.Mask") (remove_unused_layers no) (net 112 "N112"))
  (pad "18" thru_hole oval (at -2.54 -20.32 270) (size 1.7 1.7) (drill 1) (layers "*.Cu" "*.Mask") (remove_unused_layers no)
   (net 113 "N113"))
  (pad "19" thru_hole oval (at 0 -22.86 270) (size 1.7 1.7) (drill 1) (layers "*.Cu" "*.Mask") (remove_unused_layers no) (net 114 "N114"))
  (pad "20" thru_hole oval (at -2.54 -22.86 270) (size 1.7 1.7) (drill 1) (layers "*.Cu" "*.Mask") (remove_unused_layers no)
   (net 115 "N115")))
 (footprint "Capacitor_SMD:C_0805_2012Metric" (layer "B.Cu") (at 160.02 68.58 180)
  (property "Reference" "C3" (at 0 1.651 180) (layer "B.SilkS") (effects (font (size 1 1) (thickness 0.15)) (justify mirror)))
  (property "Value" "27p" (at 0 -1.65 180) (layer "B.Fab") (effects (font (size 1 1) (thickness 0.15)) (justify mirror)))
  (pad "1" smd roundrect (at -0.9375 0 180) (size 0.975 1.4) (layers "B.Cu" "B.Paste" "B.Mask") (roundrect_rratio 0.25) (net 50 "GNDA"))
  (pad "2" smd roundrect (at 0.9375 0 180) (size 0.975 1.4) (layers "B.Cu" "B.Paste" "B.Mask") (roundrect_rratio 0.25) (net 44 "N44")))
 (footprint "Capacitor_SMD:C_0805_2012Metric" (layer "B.Cu") (at 163.83 68.58)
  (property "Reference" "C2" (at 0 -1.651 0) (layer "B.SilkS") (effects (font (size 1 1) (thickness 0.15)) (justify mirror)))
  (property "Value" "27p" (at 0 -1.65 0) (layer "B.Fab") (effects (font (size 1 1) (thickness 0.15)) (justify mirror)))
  (pad "1" smd roundrect (at -0.9375 0) (size 0.975 1.4) (layers "B.Cu" "B.Paste" "B.Mask") (roundrect_rratio 0.25) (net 50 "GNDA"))
  (pad "2" smd roundrect (at 0.9375 0) (size 0.975 1.4) (layers "B.Cu" "B.Paste" "B.Mask") (roundrect_rratio 0.25) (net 43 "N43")))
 (gr_line (start 154.94 40.64) (end 157.48 38.1) (stroke (width 0.1) (type solid)) (layer "Edge.Cuts"))
 (gr_line (start 185.42 129.54) (end 157.48 129.54) (stroke (width 0.1) (type solid)) (layer "Edge.Cuts"))
 (gr_line (start 187.96 127) (end 185.42 129.54) (stroke (width 0.1) (type solid)) (layer "Edge.Cuts"))
 (gr_line (start 154.94 127) (end 154.94 40.64) (stroke (width 0.1) (type solid)) (layer "Edge.Cuts"))
 (gr_line (start 185.42 38.1) (end 187.96 40.64) (stroke (width 0.1) (type solid)) (layer "Edge.Cuts"))
 (gr_line (start 157.48 129.54) (end 154.94 127) (stroke (width 0.1) (type solid)) (layer "Edge.Cuts"))
 (gr_line (start 157.48 38.1) (end 185.42 38.1) (stroke (width 0.1) (type solid)) (layer "Edge.Cuts"))
 (gr_line (start 187.96 40.64) (end 187.96 127) (stroke (width 0.1) (type solid)) (layer "Edge.Cuts"))
 (segment (start 164.7675 65.0725) (end 164.465 64.77) (width 0.25) (layer "B.Cu") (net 43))
 (segment (start 164.7675 68.58) (end 164.7675 65.0725) (width 0.25) (layer "B.Cu") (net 43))
 (segment (start 164.7675 68.58) (end 164.719 68.6285) (width 0.25) (layer "B.Cu") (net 43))
 (segment (start 159.0825 68.58) (end 159.0825 65.2525) (width 0.25) (layer "B.Cu") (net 44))
 (segment (start 159.0825 65.2525) (end 159.565 64.77) (width 0.25) (layer "B.Cu") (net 44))
 (segment (start 159.638737 69.136237) (end 159.0825 68.58) (width 0.25) (layer "B.Cu") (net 44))
 (segment (start 167.64 121.92) (end 165.1 119.38) (width 0.25) (layer "F.Cu") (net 81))
 (segment (start 182.88 124.46) (end 184.912 122.428) (width 1) (layer "F.Cu") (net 50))
 (via (at 162.052 68.58) (size 0.8) (drill 0.4) (layers "F.Cu" "B.Cu") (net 50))
 (segment (start 160.9575 68.58) (end 162.052 68.58) (width 0.25) (layer "B.Cu") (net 50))
 (segment (start 162.052 68.58) (end 162.8925 68.58) (width 0.25) (layer "B.Cu") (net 50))
 (segment (start 182.88 121.92) (end 184.912 119.888) (width 1) (layer "B.Cu") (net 45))
 (segment (start 158.496 117.856) (end 177.8 98.552) (width 0.25) (layer "B.Cu") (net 69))
 (segment (start 158.496 122.936) (end 158.496 117.856) (width 0.25) (layer "B.Cu") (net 69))
 (segment (start 160.02 124.46) (end 158.496 122.936) (width 0.25) (layer "B.Cu") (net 69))
 (segment (start 158.496 126.492) (end 157.48 125.476) (width 0.25) (layer "B.Cu") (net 49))
 (segment (start 160.273002 126.492) (end 158.496 126.492) (width 0.25) (layer "B.Cu") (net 49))
 (segment (start 162.56 121.92) (end 161.384999 123.095001) (width 0.25) (layer "B.Cu") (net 49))
 (segment (start 161.384999 123.095001) (end 161.384999 125.380003) (width 0.25) (layer "B.Cu") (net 49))
 (segment (start 161.384999 125.380003) (end 160.273002 126.492) (width 0.25) (layer "B.Cu") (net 49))
 (segment (start 161.710001 123.610001) (end 162.56 124.46) (width 0.25) (layer "F.Cu") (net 59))
 (segment (start 161.384999 123.284999) (end 161.710001 123.610001) (width 0.25) (layer "F.Cu") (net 59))
 (segment (start 161.834999 118.654999) (end 165.1 121.92) (width 0.25) (layer "F.Cu") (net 60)))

